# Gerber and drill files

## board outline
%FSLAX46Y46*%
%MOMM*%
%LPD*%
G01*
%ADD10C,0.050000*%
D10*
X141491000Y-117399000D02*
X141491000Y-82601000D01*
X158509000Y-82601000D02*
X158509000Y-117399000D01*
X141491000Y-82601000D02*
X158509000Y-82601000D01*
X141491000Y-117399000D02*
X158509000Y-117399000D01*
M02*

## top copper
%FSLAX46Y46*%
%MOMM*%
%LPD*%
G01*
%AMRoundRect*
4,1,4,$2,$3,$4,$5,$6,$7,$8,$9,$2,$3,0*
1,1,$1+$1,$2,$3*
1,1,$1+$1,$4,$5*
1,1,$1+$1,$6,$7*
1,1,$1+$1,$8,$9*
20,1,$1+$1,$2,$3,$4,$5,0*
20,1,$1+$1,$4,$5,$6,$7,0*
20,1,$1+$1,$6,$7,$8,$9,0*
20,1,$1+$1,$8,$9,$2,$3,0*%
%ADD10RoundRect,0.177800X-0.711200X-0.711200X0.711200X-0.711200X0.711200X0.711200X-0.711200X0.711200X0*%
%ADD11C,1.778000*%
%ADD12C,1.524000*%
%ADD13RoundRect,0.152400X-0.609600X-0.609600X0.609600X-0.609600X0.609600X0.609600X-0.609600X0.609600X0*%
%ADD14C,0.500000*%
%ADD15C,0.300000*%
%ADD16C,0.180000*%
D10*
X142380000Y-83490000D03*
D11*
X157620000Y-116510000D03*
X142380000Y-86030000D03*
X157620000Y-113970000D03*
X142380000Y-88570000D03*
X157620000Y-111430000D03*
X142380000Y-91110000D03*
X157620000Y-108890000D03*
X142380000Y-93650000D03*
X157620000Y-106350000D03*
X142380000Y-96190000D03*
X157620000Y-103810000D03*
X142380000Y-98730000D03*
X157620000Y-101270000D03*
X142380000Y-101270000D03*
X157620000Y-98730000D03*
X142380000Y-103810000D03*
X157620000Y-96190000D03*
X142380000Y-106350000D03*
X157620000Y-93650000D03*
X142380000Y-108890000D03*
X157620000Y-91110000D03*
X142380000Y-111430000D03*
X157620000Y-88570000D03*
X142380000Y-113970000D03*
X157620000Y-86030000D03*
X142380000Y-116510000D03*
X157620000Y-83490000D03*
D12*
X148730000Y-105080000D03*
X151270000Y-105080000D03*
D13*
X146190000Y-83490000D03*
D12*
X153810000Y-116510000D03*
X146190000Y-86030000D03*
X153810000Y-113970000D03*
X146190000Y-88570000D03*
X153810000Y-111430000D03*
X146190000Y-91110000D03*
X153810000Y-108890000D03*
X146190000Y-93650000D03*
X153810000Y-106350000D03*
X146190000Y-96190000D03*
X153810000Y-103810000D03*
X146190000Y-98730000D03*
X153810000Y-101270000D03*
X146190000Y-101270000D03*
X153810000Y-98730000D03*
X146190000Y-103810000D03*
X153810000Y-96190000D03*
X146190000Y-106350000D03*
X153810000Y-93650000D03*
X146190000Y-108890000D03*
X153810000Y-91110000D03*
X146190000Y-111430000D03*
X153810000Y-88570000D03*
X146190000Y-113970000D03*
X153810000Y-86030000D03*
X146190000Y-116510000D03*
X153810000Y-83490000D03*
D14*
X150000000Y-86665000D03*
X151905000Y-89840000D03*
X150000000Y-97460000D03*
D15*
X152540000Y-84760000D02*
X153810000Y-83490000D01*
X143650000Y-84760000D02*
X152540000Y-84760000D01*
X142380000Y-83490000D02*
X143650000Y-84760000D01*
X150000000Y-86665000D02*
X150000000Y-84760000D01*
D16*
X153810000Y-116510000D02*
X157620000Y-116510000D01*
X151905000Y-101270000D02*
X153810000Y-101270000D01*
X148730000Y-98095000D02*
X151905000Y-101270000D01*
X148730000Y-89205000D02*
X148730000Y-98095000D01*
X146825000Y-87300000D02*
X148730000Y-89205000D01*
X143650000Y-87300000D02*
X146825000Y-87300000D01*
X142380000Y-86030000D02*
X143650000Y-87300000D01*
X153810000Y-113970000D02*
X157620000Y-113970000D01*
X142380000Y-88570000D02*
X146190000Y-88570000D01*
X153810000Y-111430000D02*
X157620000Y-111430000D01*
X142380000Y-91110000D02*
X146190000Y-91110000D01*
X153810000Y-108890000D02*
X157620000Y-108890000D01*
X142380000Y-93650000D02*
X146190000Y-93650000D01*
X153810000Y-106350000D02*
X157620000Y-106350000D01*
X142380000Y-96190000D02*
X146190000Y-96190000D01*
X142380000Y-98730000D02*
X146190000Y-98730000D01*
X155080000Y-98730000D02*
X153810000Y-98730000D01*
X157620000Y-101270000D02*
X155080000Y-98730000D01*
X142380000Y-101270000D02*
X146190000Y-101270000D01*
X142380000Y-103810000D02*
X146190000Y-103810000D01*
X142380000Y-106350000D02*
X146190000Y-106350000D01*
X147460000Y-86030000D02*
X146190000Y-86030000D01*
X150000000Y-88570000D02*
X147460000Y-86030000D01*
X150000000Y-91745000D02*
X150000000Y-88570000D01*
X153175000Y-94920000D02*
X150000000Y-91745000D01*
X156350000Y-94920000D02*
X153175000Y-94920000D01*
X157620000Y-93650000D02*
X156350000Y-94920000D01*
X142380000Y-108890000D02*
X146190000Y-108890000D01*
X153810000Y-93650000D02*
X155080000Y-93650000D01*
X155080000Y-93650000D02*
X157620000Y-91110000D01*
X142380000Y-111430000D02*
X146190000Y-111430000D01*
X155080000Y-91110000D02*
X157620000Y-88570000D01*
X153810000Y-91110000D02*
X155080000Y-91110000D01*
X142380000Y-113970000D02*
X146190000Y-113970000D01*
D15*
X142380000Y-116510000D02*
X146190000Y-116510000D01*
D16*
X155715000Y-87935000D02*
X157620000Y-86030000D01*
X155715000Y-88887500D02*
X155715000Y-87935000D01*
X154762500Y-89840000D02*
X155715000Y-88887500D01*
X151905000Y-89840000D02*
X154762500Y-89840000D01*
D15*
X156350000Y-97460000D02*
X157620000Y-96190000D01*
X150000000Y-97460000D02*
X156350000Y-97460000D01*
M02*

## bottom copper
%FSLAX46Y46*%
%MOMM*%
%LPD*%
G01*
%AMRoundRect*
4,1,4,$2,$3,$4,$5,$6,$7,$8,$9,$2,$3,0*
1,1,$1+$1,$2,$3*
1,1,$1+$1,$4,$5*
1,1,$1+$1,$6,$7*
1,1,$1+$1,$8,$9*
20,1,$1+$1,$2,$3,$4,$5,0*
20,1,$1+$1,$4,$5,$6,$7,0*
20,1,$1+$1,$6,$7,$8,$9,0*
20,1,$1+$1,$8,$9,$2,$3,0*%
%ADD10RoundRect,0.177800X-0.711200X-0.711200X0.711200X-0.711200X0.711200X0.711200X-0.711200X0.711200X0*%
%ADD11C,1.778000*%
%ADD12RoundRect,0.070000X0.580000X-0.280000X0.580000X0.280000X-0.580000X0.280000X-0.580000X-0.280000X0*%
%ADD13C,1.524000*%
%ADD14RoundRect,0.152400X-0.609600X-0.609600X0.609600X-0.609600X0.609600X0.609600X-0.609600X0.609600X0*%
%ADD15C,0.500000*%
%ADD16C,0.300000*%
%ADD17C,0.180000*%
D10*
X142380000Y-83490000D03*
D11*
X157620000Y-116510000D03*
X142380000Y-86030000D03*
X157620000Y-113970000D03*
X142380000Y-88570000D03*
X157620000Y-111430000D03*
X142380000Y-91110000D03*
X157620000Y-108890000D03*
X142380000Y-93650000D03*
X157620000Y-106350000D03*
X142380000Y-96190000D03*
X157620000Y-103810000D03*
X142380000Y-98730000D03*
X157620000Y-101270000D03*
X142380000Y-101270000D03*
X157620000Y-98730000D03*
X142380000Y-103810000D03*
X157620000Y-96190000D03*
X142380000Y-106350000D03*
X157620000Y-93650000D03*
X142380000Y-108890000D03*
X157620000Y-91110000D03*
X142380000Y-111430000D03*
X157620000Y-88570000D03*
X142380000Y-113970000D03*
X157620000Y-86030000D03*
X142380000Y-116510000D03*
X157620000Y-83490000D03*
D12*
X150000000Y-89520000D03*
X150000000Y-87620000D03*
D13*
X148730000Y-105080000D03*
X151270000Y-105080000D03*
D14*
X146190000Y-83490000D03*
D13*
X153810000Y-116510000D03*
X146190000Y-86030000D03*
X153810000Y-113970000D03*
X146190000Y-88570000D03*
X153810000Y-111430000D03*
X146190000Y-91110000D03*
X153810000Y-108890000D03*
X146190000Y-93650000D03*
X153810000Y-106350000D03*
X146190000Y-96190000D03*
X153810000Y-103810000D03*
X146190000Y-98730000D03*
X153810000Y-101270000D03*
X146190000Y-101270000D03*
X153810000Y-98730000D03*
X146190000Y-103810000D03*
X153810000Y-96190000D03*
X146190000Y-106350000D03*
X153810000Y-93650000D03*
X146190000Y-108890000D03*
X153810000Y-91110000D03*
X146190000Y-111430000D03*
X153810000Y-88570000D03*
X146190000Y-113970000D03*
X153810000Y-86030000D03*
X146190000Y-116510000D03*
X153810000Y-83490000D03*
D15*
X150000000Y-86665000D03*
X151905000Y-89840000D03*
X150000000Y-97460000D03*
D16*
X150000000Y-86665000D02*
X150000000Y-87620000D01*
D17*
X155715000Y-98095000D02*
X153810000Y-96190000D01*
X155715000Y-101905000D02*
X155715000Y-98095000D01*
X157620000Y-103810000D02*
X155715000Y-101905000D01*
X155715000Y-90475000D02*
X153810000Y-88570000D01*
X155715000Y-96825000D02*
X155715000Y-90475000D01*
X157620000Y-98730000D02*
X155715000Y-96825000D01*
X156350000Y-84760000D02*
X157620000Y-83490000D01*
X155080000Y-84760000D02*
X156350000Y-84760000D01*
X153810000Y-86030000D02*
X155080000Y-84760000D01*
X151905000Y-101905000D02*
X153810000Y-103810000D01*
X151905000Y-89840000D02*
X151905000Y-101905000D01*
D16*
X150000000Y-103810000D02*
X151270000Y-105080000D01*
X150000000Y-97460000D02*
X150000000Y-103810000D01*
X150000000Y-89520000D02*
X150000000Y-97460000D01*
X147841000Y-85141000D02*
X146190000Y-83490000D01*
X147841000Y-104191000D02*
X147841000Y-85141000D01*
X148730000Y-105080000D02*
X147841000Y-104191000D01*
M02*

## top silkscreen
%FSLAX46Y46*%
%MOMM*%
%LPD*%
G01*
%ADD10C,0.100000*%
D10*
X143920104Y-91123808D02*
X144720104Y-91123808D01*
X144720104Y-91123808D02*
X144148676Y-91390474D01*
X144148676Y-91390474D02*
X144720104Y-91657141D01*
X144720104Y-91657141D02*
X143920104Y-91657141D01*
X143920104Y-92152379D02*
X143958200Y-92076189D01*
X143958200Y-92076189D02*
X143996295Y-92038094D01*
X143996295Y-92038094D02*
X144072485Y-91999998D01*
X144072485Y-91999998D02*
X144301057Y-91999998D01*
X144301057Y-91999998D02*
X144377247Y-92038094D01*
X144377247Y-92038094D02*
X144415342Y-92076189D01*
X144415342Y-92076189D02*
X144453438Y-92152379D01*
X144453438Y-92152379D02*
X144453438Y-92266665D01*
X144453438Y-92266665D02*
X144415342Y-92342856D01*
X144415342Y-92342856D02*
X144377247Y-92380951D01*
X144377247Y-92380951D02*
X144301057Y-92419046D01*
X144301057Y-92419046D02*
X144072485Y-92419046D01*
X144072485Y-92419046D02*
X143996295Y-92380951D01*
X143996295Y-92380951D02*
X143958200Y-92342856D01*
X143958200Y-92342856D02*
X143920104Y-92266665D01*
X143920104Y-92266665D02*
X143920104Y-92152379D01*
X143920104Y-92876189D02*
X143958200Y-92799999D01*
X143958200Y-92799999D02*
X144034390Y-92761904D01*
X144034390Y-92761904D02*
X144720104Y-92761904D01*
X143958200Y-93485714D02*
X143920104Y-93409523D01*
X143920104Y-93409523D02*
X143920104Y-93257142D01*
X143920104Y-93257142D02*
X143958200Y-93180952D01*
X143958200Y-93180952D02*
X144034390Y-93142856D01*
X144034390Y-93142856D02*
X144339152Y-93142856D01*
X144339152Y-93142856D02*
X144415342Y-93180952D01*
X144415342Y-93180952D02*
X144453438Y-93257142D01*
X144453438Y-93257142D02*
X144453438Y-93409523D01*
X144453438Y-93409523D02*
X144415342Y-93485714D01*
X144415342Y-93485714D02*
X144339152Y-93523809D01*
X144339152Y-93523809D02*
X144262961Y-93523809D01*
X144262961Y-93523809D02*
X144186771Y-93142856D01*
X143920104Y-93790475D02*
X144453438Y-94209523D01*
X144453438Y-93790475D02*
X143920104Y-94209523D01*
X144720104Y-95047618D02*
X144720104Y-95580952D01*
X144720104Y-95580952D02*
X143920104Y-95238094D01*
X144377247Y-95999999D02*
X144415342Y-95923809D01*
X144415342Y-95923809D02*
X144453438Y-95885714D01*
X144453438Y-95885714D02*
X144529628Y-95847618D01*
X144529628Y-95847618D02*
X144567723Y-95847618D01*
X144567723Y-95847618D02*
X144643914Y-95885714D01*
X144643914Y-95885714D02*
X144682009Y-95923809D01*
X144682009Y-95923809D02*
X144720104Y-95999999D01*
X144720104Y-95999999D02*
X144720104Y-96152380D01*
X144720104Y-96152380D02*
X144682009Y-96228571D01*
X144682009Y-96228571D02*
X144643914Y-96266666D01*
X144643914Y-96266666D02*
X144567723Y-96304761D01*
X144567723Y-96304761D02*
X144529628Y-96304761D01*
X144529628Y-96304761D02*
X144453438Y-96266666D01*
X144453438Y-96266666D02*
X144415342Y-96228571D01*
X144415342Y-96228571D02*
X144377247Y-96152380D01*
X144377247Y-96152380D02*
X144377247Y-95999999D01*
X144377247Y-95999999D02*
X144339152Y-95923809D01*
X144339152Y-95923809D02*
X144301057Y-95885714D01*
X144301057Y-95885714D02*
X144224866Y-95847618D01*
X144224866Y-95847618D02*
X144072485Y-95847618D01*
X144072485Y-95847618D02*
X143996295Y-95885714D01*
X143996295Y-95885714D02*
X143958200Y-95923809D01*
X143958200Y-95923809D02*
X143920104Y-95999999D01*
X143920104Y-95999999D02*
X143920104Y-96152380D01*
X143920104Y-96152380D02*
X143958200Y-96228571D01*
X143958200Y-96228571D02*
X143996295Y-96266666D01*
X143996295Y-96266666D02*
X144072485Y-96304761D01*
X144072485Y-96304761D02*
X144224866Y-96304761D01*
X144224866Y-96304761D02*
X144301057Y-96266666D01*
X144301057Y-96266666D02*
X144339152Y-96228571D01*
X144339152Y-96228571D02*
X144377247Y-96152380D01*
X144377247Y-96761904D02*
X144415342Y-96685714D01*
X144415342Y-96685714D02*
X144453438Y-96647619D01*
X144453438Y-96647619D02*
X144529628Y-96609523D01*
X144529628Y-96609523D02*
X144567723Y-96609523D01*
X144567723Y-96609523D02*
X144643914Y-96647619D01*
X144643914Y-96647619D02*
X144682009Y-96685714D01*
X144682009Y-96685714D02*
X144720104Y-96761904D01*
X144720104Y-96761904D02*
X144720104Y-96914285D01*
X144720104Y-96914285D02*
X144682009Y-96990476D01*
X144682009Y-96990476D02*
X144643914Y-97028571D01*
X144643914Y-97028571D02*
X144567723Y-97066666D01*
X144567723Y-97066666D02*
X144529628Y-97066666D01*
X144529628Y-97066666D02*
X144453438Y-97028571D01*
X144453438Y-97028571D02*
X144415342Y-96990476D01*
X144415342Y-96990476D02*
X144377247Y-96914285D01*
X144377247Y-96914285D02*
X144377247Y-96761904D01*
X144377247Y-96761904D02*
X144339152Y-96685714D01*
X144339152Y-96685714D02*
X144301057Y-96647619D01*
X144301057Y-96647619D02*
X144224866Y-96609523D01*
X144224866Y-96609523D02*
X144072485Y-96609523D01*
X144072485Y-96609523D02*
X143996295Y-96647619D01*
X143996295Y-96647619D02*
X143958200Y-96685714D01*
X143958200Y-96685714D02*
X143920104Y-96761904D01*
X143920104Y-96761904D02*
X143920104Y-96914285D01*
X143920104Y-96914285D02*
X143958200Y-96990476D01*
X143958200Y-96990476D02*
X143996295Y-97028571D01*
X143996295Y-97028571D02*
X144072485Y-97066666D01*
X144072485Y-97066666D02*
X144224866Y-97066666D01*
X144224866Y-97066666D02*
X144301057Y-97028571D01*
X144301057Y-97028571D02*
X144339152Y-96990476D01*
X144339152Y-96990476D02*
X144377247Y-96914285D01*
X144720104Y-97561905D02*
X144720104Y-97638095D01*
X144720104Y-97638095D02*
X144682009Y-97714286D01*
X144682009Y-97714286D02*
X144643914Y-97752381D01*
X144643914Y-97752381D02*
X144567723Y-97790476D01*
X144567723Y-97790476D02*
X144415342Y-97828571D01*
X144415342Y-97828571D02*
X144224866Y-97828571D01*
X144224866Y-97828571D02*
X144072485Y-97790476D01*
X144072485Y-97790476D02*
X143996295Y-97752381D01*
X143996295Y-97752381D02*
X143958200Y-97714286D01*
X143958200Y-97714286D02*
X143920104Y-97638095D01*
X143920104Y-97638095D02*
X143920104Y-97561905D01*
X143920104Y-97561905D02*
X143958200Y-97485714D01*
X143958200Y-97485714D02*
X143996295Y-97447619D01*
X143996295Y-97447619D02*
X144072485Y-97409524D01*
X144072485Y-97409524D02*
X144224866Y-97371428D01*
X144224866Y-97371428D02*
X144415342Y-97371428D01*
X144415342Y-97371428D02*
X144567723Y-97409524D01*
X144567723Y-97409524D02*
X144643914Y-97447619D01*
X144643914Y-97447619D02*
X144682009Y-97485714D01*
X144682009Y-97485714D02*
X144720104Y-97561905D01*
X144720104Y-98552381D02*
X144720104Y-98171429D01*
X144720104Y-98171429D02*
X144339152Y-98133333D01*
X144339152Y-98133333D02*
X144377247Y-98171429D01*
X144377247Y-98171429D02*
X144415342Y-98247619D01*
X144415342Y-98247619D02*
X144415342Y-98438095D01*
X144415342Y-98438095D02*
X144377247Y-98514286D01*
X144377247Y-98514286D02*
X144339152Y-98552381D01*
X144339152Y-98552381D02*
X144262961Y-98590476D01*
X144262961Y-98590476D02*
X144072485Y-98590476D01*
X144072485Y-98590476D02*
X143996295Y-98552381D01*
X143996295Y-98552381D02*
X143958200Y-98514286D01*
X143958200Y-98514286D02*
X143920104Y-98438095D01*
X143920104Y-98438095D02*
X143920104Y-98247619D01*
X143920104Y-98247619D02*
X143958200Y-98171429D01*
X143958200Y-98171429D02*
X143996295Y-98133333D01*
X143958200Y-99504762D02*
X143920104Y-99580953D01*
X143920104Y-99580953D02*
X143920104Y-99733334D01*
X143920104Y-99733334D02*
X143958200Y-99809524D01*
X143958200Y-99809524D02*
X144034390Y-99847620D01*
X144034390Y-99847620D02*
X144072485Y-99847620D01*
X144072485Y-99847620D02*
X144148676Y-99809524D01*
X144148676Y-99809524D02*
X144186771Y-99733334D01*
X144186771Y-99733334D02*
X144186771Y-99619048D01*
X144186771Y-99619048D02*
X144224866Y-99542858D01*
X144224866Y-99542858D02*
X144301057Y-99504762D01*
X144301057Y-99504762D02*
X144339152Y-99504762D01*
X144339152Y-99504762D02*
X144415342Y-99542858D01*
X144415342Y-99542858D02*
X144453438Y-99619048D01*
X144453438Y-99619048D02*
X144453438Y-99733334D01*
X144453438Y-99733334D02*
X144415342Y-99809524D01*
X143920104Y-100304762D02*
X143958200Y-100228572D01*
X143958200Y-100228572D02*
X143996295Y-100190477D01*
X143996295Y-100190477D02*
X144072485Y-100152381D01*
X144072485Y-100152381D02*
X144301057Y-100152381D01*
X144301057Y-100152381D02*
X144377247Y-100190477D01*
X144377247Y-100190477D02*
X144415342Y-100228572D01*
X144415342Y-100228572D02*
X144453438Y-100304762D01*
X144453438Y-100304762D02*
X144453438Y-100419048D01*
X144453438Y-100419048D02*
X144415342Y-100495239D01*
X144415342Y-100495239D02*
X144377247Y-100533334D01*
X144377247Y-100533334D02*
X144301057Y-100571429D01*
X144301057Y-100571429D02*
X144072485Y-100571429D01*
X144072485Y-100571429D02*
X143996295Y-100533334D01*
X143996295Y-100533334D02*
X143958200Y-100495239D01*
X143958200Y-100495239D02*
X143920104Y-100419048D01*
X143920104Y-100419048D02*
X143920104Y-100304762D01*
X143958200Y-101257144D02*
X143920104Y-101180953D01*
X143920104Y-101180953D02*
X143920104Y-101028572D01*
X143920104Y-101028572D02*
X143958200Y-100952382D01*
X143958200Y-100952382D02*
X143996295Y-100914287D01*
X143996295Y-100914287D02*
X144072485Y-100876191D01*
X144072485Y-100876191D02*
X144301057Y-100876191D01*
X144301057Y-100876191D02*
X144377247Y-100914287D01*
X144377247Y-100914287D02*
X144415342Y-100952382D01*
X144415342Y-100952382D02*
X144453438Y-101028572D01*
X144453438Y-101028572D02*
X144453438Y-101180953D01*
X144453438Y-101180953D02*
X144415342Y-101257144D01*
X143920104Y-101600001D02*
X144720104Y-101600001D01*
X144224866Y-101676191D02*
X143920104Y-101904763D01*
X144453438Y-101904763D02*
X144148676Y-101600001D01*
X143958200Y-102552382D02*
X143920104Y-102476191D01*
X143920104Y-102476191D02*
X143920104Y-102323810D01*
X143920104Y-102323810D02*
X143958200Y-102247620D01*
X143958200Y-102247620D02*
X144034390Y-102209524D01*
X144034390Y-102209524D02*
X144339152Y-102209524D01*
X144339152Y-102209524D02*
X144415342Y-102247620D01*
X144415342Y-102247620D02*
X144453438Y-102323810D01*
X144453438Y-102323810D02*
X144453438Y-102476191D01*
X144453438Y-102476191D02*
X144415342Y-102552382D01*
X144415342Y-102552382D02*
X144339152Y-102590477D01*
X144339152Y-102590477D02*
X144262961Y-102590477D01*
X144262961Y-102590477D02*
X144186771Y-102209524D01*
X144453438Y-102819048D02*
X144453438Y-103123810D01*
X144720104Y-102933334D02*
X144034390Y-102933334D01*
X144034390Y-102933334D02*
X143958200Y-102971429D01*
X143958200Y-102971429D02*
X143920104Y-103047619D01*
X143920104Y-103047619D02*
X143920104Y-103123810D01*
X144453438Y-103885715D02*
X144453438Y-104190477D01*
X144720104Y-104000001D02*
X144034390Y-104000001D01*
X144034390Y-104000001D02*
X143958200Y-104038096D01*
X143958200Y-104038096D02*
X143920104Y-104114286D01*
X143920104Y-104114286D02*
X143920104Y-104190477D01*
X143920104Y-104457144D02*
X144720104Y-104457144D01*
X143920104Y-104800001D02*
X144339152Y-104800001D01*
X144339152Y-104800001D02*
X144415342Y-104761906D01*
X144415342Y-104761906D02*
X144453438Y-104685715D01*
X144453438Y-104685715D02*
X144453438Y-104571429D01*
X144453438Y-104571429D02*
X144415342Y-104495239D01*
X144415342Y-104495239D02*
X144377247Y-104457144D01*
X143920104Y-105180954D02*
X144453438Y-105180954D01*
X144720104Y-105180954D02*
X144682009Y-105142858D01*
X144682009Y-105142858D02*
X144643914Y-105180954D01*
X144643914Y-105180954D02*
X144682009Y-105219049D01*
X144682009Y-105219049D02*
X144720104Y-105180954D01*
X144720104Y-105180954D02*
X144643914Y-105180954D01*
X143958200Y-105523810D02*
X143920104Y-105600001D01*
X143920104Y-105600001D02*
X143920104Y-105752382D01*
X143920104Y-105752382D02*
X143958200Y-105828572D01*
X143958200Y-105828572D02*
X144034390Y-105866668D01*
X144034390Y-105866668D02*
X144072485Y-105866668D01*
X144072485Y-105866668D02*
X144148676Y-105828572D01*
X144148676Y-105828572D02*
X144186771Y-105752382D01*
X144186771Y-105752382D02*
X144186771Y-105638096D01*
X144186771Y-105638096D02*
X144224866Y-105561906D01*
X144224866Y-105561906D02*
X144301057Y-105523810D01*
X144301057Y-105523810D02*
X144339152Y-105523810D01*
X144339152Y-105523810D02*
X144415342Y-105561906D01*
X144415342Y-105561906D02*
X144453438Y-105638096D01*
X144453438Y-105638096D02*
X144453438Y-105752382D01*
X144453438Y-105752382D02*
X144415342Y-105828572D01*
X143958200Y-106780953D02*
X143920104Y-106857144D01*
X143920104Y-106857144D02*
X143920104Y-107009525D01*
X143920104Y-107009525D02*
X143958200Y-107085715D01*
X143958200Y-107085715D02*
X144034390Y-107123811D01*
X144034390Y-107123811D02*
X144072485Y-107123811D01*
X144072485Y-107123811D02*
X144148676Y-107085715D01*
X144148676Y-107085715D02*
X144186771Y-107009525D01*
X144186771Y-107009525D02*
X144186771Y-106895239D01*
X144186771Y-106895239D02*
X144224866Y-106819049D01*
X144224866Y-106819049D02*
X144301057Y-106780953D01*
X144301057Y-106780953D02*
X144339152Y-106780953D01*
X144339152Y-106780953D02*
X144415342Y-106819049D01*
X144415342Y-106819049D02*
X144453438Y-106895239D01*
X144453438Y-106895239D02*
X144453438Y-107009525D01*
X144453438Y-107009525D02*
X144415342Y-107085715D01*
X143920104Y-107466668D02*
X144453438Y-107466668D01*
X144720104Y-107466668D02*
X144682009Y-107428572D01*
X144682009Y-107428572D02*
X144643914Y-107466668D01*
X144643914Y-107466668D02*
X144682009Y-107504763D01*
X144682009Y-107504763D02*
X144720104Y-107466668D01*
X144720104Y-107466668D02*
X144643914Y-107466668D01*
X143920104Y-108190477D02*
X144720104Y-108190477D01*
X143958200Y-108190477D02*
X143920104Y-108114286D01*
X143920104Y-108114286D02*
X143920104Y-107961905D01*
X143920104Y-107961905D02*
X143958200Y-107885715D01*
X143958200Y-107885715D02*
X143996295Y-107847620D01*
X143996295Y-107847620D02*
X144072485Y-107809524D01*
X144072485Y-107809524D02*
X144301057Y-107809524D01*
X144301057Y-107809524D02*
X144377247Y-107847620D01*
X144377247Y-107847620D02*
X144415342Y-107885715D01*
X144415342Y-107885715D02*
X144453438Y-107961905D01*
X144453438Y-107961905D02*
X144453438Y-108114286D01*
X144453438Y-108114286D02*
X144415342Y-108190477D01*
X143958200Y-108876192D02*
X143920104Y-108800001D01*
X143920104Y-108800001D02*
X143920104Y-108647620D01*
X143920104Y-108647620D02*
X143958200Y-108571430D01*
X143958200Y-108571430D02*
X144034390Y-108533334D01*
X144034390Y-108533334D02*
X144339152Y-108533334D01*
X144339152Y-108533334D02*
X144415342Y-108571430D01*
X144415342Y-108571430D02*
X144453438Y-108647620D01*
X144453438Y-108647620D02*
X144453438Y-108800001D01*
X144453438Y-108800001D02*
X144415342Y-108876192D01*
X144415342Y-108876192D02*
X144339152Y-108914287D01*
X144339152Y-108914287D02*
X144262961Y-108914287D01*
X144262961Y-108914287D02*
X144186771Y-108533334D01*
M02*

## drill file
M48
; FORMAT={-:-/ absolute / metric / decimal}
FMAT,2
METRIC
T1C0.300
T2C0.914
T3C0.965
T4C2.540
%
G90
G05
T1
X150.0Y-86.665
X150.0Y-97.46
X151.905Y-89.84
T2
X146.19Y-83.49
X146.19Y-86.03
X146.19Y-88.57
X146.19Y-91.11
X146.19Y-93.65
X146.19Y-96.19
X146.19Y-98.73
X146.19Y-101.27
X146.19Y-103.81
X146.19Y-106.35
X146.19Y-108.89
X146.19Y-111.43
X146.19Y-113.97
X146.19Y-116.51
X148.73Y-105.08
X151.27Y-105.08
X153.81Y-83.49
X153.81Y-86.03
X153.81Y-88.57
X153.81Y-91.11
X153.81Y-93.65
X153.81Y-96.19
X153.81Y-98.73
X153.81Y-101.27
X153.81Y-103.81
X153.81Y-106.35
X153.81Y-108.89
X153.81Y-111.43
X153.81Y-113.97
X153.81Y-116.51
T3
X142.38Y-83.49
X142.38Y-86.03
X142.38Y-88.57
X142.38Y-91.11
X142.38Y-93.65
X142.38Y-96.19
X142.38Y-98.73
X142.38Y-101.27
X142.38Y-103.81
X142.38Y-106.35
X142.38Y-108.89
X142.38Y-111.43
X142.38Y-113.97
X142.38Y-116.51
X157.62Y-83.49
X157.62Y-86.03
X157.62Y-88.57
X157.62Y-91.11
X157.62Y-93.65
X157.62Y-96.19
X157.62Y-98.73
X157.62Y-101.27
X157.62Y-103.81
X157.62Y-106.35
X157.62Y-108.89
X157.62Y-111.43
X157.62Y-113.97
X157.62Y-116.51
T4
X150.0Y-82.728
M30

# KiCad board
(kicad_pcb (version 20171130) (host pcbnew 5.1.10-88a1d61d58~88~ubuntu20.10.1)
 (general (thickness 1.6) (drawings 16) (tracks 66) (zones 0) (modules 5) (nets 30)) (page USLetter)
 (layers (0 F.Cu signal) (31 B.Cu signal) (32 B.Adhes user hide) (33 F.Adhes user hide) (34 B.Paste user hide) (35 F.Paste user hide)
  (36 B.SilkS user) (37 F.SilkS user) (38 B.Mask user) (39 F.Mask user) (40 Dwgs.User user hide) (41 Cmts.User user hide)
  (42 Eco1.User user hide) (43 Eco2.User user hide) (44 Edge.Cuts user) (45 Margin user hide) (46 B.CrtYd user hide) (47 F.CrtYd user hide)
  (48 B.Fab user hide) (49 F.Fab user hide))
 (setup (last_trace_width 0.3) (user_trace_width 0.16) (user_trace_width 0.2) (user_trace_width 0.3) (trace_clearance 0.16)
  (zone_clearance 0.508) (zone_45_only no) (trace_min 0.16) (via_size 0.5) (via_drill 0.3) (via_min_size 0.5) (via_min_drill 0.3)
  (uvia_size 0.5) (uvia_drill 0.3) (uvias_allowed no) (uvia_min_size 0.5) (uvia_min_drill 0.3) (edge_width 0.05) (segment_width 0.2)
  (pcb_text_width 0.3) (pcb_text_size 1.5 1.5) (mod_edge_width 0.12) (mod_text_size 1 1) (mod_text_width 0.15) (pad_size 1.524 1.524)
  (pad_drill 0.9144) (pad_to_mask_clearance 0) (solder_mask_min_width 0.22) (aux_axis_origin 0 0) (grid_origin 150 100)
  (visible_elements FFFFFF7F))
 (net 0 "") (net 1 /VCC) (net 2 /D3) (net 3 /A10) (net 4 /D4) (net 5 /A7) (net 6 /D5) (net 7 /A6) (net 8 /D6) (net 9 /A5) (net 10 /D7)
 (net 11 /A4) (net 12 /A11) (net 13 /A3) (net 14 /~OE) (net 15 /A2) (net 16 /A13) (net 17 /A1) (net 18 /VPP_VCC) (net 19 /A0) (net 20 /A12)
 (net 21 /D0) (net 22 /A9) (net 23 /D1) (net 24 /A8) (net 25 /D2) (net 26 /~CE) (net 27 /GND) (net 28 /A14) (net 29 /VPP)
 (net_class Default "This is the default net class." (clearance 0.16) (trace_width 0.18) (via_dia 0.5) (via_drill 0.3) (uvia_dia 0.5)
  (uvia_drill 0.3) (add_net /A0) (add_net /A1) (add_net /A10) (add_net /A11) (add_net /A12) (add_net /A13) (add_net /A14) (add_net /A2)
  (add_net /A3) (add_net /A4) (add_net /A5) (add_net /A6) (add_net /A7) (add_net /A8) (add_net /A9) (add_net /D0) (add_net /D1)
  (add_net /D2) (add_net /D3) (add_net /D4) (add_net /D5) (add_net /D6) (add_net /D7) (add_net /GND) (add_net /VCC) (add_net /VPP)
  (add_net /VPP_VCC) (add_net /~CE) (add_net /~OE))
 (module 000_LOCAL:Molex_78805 (layer F.Cu) (at 150 100)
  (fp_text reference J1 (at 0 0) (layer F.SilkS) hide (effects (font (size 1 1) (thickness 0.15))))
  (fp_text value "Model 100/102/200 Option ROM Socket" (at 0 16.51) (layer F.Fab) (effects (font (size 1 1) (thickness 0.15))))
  (pad 1 thru_hole roundrect (at -7.62 -16.51) (size 1.778 1.778) (drill 0.9652) (layers *.Cu *.Mask) (roundrect_rratio 0.1) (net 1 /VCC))
  (pad 15 thru_hole circle (at 7.62 16.51) (size 1.778 1.778) (drill 0.9652) (layers *.Cu *.Mask) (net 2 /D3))
  (pad 2 thru_hole circle (at -7.62 -13.97) (size 1.778 1.778) (drill 0.9652) (layers *.Cu *.Mask) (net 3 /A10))
  (pad 16 thru_hole circle (at 7.62 13.97) (size 1.778 1.778) (drill 0.9652) (layers *.Cu *.Mask) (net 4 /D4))
  (pad 3 thru_hole circle (at -7.62 -11.43) (size 1.778 1.778) (drill 0.9652) (layers *.Cu *.Mask) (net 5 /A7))
  (pad 17 thru_hole circle (at 7.62 11.43) (size 1.778 1.778) (drill 0.9652) (layers *.Cu *.Mask) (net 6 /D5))
  (pad 4 thru_hole circle (at -7.62 -8.89) (size 1.778 1.778) (drill 0.9652) (layers *.Cu *.Mask) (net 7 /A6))
  (pad 18 thru_hole circle (at 7.62 8.89) (size 1.778 1.778) (drill 0.9652) (layers *.Cu *.Mask) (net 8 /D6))
  (pad 5 thru_hole circle (at -7.62 -6.35) (size 1.778 1.778) (drill 0.9652) (layers *.Cu *.Mask) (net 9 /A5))
  (pad 19 thru_hole circle (at 7.62 6.35) (size 1.778 1.778) (drill 0.9652) (layers *.Cu *.Mask) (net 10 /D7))
  (pad 6 thru_hole circle (at -7.62 -3.81) (size 1.778 1.778) (drill 0.9652) (layers *.Cu *.Mask) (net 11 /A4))
  (pad 20 thru_hole circle (at 7.62 3.81) (size 1.778 1.778) (drill 0.9652) (layers *.Cu *.Mask) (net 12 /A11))
  (pad 7 thru_hole circle (at -7.62 -1.27) (size 1.778 1.778) (drill 0.9652) (layers *.Cu *.Mask) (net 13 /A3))
  (pad 21 thru_hole circle (at 7.62 1.27) (size 1.778 1.778) (drill 0.9652) (layers *.Cu *.Mask) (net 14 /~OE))
  (pad 8 thru_hole circle (at -7.62 1.27) (size 1.778 1.778) (drill 0.9652) (layers *.Cu *.Mask) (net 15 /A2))
  (pad 22 thru_hole circle (at 7.62 -1.27) (size 1.778 1.778) (drill 0.9652) (layers *.Cu *.Mask) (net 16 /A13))
  (pad 9 thru_hole circle (at -7.62 3.81) (size 1.778 1.778) (drill 0.9652) (layers *.Cu *.Mask) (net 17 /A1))
  (pad 23 thru_hole circle (at 7.62 -3.81) (size 1.778 1.778) (drill 0.9652) (layers *.Cu *.Mask) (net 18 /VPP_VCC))
  (pad 10 thru_hole circle (at -7.62 6.35) (size 1.778 1.778) (drill 0.9652) (layers *.Cu *.Mask) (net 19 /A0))
  (pad 24 thru_hole circle (at 7.62 -6.35) (size 1.778 1.778) (drill 0.9652) (layers *.Cu *.Mask) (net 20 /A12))
  (pad 11 thru_hole circle (at -7.62 8.89) (size 1.778 1.778) (drill 0.9652) (layers *.Cu *.Mask) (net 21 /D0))
  (pad 25 thru_hole circle (at 7.62 -8.89) (size 1.778 1.778) (drill 0.9652) (layers *.Cu *.Mask) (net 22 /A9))
  (pad 12 thru_hole circle (at -7.62 11.43) (size 1.778 1.778) (drill 0.9652) (layers *.Cu *.Mask) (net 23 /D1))
  (pad 26 thru_hole circle (at 7.62 -11.43) (size 1.778 1.778) (drill 0.9652) (layers *.Cu *.Mask) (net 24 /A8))
  (pad 13 thru_hole circle (at -7.62 13.97) (size 1.778 1.778) (drill 0.9652) (layers *.Cu *.Mask) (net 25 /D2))
  (pad 27 thru_hole circle (at 7.62 -13.97) (size 1.778 1.778) (drill 0.9652) (layers *.Cu *.Mask) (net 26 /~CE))
  (pad 14 thru_hole circle (at -7.62 16.51) (size 1.778 1.778) (drill 0.9652) (layers *.Cu *.Mask) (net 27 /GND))
  (pad 28 thru_hole circle (at 7.62 -16.51) (size 1.778 1.778) (drill 0.9652) (layers *.Cu *.Mask) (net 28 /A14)))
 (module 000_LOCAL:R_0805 (layer B.Cu) (at 150 88.57 90)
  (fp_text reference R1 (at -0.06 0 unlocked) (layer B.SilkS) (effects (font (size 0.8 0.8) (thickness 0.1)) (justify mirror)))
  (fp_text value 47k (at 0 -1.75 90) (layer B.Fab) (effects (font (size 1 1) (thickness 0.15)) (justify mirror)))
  (pad 1 smd roundrect (at -0.95 0 90) (size 0.7 1.3) (layers B.Cu B.Paste B.Mask) (roundrect_rratio 0.1) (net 18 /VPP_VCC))
  (pad 2 smd roundrect (at 0.95 0 90) (size 0.7 1.3) (layers B.Cu B.Paste B.Mask) (roundrect_rratio 0.1) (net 1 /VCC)))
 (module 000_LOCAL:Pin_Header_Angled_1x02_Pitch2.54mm (layer B.Cu) (at 148.73 105.08 270)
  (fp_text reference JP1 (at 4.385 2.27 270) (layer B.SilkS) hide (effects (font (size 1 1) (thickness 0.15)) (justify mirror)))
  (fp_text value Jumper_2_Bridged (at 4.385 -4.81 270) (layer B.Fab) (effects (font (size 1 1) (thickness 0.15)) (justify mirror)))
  (pad 1 thru_hole circle (at 0 0 270) (size 1.524 1.524) (drill 0.9144) (layers *.Cu *.Mask) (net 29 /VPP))
  (pad 2 thru_hole circle (at 0 -2.54 270) (size 1.524 1.524) (drill 0.9144) (layers *.Cu *.Mask) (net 18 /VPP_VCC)))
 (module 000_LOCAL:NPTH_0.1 (layer F.Cu) (at 150 82.728)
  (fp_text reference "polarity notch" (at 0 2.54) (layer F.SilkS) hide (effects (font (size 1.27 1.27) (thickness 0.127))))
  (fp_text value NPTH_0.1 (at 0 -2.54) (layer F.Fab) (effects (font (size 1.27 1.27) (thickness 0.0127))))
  (pad "" np_thru_hole circle (at 0 0) (size 2.54 2.54) (drill 2.54) (layers *.Cu *.Mask)))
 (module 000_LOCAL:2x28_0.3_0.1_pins (layer F.Cu) (at 150 100)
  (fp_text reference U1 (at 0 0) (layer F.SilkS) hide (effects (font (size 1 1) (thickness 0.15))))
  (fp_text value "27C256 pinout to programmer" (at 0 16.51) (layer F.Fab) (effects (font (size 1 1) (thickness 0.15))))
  (pad 1 thru_hole roundrect (at -3.81 -16.51) (size 1.524 1.524) (drill 0.9144) (layers *.Cu *.Mask) (roundrect_rratio 0.1) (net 29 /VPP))
  (pad 15 thru_hole circle (at 3.81 16.51) (size 1.524 1.524) (drill 0.9144) (layers *.Cu *.Mask) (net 2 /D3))
  (pad 2 thru_hole circle (at -3.81 -13.97) (size 1.524 1.524) (drill 0.9144) (layers *.Cu *.Mask) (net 20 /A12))
  (pad 16 thru_hole circle (at 3.81 13.97) (size 1.524 1.524) (drill 0.9144) (layers *.Cu *.Mask) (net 4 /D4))
  (pad 3 thru_hole circle (at -3.81 -11.43) (size 1.524 1.524) (drill 0.9144) (layers *.Cu *.Mask) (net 5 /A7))
  (pad 17 thru_hole circle (at 3.81 11.43) (size 1.524 1.524) (drill 0.9144) (layers *.Cu *.Mask) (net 6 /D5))
  (pad 4 thru_hole circle (at -3.81 -8.89) (size 1.524 1.524) (drill 0.9144) (layers *.Cu *.Mask) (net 7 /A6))
  (pad 18 thru_hole circle (at 3.81 8.89) (size 1.524 1.524) (drill 0.9144) (layers *.Cu *.Mask) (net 8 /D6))
  (pad 5 thru_hole circle (at -3.81 -6.35) (size 1.524 1.524) (drill 0.9144) (layers *.Cu *.Mask) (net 9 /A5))
  (pad 19 thru_hole circle (at 3.81 6.35) (size 1.524 1.524) (drill 0.9144) (layers *.Cu *.Mask) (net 10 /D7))
  (pad 6 thru_hole circle (at -3.81 -3.81) (size 1.524 1.524) (drill 0.9144) (layers *.Cu *.Mask) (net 11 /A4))
  (pad 20 thru_hole circle (at 3.81 3.81) (size 1.524 1.524) (drill 0.9144) (layers *.Cu *.Mask) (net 26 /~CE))
  (pad 7 thru_hole circle (at -3.81 -1.27) (size 1.524 1.524) (drill 0.9144) (layers *.Cu *.Mask) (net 13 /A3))
  (pad 21 thru_hole circle (at 3.81 1.27) (size 1.524 1.524) (drill 0.9144) (layers *.Cu *.Mask) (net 3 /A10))
  (pad 8 thru_hole circle (at -3.81 1.27) (size 1.524 1.524) (drill 0.9144) (layers *.Cu *.Mask) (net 15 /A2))
  (pad 22 thru_hole circle (at 3.81 -1.27) (size 1.524 1.524) (drill 0.9144) (layers *.Cu *.Mask) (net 14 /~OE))
  (pad 9 thru_hole circle (at -3.81 3.81) (size 1.524 1.524) (drill 0.9144) (layers *.Cu *.Mask) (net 17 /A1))
  (pad 23 thru_hole circle (at 3.81 -3.81) (size 1.524 1.524) (drill 0.9144) (layers *.Cu *.Mask) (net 12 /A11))
  (pad 10 thru_hole circle (at -3.81 6.35) (size 1.524 1.524) (drill 0.9144) (layers *.Cu *.Mask) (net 19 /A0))
  (pad 24 thru_hole circle (at 3.81 -6.35) (size 1.524 1.524) (drill 0.9144) (layers *.Cu *.Mask) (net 22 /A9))
  (pad 11 thru_hole circle (at -3.81 8.89) (size 1.524 1.524) (drill 0.9144) (layers *.Cu *.Mask) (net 21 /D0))
  (pad 25 thru_hole circle (at 3.81 -8.89) (size 1.524 1.524) (drill 0.9144) (layers *.Cu *.Mask) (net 24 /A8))
  (pad 12 thru_hole circle (at -3.81 11.43) (size 1.524 1.524) (drill 0.9144) (layers *.Cu *.Mask) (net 23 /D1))
  (pad 26 thru_hole circle (at 3.81 -11.43) (size 1.524 1.524) (drill 0.9144) (layers *.Cu *.Mask) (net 16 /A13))
  (pad 13 thru_hole circle (at -3.81 13.97) (size 1.524 1.524) (drill 0.9144) (layers *.Cu *.Mask) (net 25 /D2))
  (pad 27 thru_hole circle (at 3.81 -13.97) (size 1.524 1.524) (drill 0.9144) (layers *.Cu *.Mask) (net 28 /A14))
  (pad 14 thru_hole circle (at -3.81 16.51) (size 1.524 1.524) (drill 0.9144) (layers *.Cu *.Mask) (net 27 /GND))
  (pad 28 thru_hole circle (at 3.81 -16.51) (size 1.524 1.524) (drill 0.9144) (layers *.Cu *.Mask) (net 1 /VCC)))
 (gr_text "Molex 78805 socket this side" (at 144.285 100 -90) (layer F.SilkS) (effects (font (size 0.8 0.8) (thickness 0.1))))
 (gr_line (start 141.491 117.399) (end 141.491 82.601) (layer Edge.Cuts) (width 0.05))
 (gr_line (start 158.509 82.601) (end 158.509 117.399) (layer Edge.Cuts) (width 0.05))
 (gr_line (start 141.491 82.601) (end 158.509 82.601) (layer Edge.Cuts) (width 0.05))
 (gr_line (start 141.491 117.399) (end 158.509 117.399) (layer Edge.Cuts) (width 0.05))
 (via (at 150 86.665) (size 0.5) (drill 0.3) (layers F.Cu B.Cu) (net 1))
 (segment (start 152.54 84.76) (end 153.81 83.49) (width 0.3) (layer F.Cu) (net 1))
 (segment (start 143.65 84.76) (end 152.54 84.76) (width 0.3) (layer F.Cu) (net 1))
 (segment (start 142.38 83.49) (end 143.65 84.76) (width 0.3) (layer F.Cu) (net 1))
 (segment (start 150 86.665) (end 150 84.76) (width 0.3) (layer F.Cu) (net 1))
 (segment (start 150 86.665) (end 150 87.62) (width 0.3) (layer B.Cu) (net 1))
 (segment (start 153.81 116.51) (end 157.62 116.51) (width 0.18) (layer F.Cu) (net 2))
 (segment (start 151.905 101.27) (end 153.81 101.27) (width 0.18) (layer F.Cu) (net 3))
 (segment (start 148.73 98.095) (end 151.905 101.27) (width 0.18) (layer F.Cu) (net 3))
 (segment (start 148.73 89.205) (end 148.73 98.095) (width 0.18) (layer F.Cu) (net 3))
 (segment (start 146.825 87.3) (end 148.73 89.205) (width 0.18) (layer F.Cu) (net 3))
 (segment (start 143.65 87.3) (end 146.825 87.3) (width 0.18) (layer F.Cu) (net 3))
 (segment (start 142.38 86.03) (end 143.65 87.3) (width 0.18) (layer F.Cu) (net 3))
 (segment (start 153.81 113.97) (end 157.62 113.97) (width 0.18) (layer F.Cu) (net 4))
 (segment (start 142.38 88.57) (end 146.19 88.57) (width 0.18) (layer F.Cu) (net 5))
 (segment (start 153.81 111.43) (end 157.62 111.43) (width 0.18) (layer F.Cu) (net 6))
 (segment (start 142.38 91.11) (end 146.19 91.11) (width 0.18) (layer F.Cu) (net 7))
 (segment (start 153.81 108.89) (end 157.62 108.89) (width 0.18) (layer F.Cu) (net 8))
 (segment (start 142.38 93.65) (end 146.19 93.65) (width 0.18) (layer F.Cu) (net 9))
 (segment (start 153.81 106.35) (end 157.62 106.35) (width 0.18) (layer F.Cu) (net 10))
 (segment (start 142.38 96.19) (end 146.19 96.19) (width 0.18) (layer F.Cu) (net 11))
 (segment (start 155.715 98.095) (end 153.81 96.19) (width 0.18) (layer B.Cu) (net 12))
 (segment (start 155.715 101.905) (end 155.715 98.095) (width 0.18) (layer B.Cu) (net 12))
 (segment (start 157.62 103.81) (end 155.715 101.905) (width 0.18) (layer B.Cu) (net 12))
 (segment (start 142.38 98.73) (end 146.19 98.73) (width 0.18) (layer F.Cu) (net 13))
 (segment (start 155.08 98.73) (end 153.81 98.73) (width 0.18) (layer F.Cu) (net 14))
 (segment (start 157.62 101.27) (end 155.08 98.73) (width 0.18) (layer F.Cu) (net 14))
 (segment (start 142.38 101.27) (end 146.19 101.27) (width 0.18) (layer F.Cu) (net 15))
 (segment (start 155.715 90.475) (end 153.81 88.57) (width 0.18) (layer B.Cu) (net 16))
 (segment (start 155.715 96.825) (end 155.715 90.475) (width 0.18) (layer B.Cu) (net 16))
 (segment (start 157.62 98.73) (end 155.715 96.825) (width 0.18) (layer B.Cu) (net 16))
 (segment (start 142.38 103.81) (end 146.19 103.81) (width 0.18) (layer F.Cu) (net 17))
 (segment (start 142.38 106.35) (end 146.19 106.35) (width 0.18) (layer F.Cu) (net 19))
 (segment (start 147.46 86.03) (end 146.19 86.03) (width 0.18) (layer F.Cu) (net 20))
 (segment (start 150 88.57) (end 147.46 86.03) (width 0.18) (layer F.Cu) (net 20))
 (segment (start 150 91.745) (end 150 88.57) (width 0.18) (layer F.Cu) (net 20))
 (segment (start 153.175 94.92) (end 150 91.745) (width 0.18) (layer F.Cu) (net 20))
 (segment (start 156.35 94.92) (end 153.175 94.92) (width 0.18) (layer F.Cu) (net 20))
 (segment (start 157.62 93.65) (end 156.35 94.92) (width 0.18) (layer F.Cu) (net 20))
 (segment (start 142.38 108.89) (end 146.19 108.89) (width 0.18) (layer F.Cu) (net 21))
 (segment (start 153.81 93.65) (end 155.08 93.65) (width 0.18) (layer F.Cu) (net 22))
 (segment (start 155.08 93.65) (end 157.62 91.11) (width 0.18) (layer F.Cu) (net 22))
 (segment (start 142.38 111.43) (end 146.19 111.43) (width 0.18) (layer F.Cu) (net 23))
 (segment (start 155.08 91.11) (end 157.62 88.57) (width 0.18) (layer F.Cu) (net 24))
 (segment (start 153.81 91.11) (end 155.08 91.11) (width 0.18) (layer F.Cu) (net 24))
 (segment (start 142.38 113.97) (end 146.19 113.97) (width 0.18) (layer F.Cu) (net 25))
 (segment (start 142.38 116.51) (end 146.19 116.51) (width 0.3) (layer F.Cu) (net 27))
 (segment (start 156.35 84.76) (end 157.62 83.49) (width 0.18) (layer B.Cu) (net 28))
 (segment (start 155.08 84.76) (end 156.35 84.76) (width 0.18) (layer B.Cu) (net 28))
 (segment (start 153.81 86.03) (end 155.08 84.76) (width 0.18) (layer B.Cu) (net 28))
 (segment (start 151.905 101.905) (end 153.81 103.81) (width 0.18) (layer B.Cu) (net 26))
 (segment (start 151.905 89.84) (end 151.905 101.905) (width 0.18) (layer B.Cu) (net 26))
 (via (at 151.905 89.84) (size 0.5) (drill 0.3) (layers F.Cu B.Cu) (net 26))
 (segment (start 155.715 87.935) (end 157.62 86.03) (width 0.18) (layer F.Cu) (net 26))
 (segment (start 155.715 88.8875) (end 155.715 87.935) (width 0.18) (layer F.Cu) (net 26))
 (segment (start 154.7625 89.84) (end 155.715 88.8875) (width 0.18) (layer F.Cu) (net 26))
 (segment (start 151.905 89.84) (end 154.7625 89.84) (width 0.18) (layer F.Cu) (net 26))
 (via (at 150 97.46) (size 0.5) (drill 0.3) (layers F.Cu B.Cu) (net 18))
 (segment (start 156.35 97.46) (end 157.62 96.19) (width 0.3) (layer F.Cu) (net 18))
 (segment (start 150 97.46) (end 156.35 97.46) (width 0.3) (layer F.Cu) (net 18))
 (segment (start 150 103.81) (end 151.27 105.08) (width 0.3) (layer B.Cu) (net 18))
 (segment (start 150 97.46) (end 150 103.81) (width 0.3) (layer B.Cu) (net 18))
 (segment (start 150 89.52) (end 150 97.46) (width 0.3) (layer B.Cu) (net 18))
 (segment (start 147.841 85.141) (end 146.19 83.49) (width 0.3) (layer B.Cu) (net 29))
 (segment (start 147.841 104.191) (end 147.841 85.141) (width 0.3) (layer B.Cu) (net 29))
 (segment (start 148.73 105.08) (end 147.841 104.191) (width 0.3) (layer B.Cu) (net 29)))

